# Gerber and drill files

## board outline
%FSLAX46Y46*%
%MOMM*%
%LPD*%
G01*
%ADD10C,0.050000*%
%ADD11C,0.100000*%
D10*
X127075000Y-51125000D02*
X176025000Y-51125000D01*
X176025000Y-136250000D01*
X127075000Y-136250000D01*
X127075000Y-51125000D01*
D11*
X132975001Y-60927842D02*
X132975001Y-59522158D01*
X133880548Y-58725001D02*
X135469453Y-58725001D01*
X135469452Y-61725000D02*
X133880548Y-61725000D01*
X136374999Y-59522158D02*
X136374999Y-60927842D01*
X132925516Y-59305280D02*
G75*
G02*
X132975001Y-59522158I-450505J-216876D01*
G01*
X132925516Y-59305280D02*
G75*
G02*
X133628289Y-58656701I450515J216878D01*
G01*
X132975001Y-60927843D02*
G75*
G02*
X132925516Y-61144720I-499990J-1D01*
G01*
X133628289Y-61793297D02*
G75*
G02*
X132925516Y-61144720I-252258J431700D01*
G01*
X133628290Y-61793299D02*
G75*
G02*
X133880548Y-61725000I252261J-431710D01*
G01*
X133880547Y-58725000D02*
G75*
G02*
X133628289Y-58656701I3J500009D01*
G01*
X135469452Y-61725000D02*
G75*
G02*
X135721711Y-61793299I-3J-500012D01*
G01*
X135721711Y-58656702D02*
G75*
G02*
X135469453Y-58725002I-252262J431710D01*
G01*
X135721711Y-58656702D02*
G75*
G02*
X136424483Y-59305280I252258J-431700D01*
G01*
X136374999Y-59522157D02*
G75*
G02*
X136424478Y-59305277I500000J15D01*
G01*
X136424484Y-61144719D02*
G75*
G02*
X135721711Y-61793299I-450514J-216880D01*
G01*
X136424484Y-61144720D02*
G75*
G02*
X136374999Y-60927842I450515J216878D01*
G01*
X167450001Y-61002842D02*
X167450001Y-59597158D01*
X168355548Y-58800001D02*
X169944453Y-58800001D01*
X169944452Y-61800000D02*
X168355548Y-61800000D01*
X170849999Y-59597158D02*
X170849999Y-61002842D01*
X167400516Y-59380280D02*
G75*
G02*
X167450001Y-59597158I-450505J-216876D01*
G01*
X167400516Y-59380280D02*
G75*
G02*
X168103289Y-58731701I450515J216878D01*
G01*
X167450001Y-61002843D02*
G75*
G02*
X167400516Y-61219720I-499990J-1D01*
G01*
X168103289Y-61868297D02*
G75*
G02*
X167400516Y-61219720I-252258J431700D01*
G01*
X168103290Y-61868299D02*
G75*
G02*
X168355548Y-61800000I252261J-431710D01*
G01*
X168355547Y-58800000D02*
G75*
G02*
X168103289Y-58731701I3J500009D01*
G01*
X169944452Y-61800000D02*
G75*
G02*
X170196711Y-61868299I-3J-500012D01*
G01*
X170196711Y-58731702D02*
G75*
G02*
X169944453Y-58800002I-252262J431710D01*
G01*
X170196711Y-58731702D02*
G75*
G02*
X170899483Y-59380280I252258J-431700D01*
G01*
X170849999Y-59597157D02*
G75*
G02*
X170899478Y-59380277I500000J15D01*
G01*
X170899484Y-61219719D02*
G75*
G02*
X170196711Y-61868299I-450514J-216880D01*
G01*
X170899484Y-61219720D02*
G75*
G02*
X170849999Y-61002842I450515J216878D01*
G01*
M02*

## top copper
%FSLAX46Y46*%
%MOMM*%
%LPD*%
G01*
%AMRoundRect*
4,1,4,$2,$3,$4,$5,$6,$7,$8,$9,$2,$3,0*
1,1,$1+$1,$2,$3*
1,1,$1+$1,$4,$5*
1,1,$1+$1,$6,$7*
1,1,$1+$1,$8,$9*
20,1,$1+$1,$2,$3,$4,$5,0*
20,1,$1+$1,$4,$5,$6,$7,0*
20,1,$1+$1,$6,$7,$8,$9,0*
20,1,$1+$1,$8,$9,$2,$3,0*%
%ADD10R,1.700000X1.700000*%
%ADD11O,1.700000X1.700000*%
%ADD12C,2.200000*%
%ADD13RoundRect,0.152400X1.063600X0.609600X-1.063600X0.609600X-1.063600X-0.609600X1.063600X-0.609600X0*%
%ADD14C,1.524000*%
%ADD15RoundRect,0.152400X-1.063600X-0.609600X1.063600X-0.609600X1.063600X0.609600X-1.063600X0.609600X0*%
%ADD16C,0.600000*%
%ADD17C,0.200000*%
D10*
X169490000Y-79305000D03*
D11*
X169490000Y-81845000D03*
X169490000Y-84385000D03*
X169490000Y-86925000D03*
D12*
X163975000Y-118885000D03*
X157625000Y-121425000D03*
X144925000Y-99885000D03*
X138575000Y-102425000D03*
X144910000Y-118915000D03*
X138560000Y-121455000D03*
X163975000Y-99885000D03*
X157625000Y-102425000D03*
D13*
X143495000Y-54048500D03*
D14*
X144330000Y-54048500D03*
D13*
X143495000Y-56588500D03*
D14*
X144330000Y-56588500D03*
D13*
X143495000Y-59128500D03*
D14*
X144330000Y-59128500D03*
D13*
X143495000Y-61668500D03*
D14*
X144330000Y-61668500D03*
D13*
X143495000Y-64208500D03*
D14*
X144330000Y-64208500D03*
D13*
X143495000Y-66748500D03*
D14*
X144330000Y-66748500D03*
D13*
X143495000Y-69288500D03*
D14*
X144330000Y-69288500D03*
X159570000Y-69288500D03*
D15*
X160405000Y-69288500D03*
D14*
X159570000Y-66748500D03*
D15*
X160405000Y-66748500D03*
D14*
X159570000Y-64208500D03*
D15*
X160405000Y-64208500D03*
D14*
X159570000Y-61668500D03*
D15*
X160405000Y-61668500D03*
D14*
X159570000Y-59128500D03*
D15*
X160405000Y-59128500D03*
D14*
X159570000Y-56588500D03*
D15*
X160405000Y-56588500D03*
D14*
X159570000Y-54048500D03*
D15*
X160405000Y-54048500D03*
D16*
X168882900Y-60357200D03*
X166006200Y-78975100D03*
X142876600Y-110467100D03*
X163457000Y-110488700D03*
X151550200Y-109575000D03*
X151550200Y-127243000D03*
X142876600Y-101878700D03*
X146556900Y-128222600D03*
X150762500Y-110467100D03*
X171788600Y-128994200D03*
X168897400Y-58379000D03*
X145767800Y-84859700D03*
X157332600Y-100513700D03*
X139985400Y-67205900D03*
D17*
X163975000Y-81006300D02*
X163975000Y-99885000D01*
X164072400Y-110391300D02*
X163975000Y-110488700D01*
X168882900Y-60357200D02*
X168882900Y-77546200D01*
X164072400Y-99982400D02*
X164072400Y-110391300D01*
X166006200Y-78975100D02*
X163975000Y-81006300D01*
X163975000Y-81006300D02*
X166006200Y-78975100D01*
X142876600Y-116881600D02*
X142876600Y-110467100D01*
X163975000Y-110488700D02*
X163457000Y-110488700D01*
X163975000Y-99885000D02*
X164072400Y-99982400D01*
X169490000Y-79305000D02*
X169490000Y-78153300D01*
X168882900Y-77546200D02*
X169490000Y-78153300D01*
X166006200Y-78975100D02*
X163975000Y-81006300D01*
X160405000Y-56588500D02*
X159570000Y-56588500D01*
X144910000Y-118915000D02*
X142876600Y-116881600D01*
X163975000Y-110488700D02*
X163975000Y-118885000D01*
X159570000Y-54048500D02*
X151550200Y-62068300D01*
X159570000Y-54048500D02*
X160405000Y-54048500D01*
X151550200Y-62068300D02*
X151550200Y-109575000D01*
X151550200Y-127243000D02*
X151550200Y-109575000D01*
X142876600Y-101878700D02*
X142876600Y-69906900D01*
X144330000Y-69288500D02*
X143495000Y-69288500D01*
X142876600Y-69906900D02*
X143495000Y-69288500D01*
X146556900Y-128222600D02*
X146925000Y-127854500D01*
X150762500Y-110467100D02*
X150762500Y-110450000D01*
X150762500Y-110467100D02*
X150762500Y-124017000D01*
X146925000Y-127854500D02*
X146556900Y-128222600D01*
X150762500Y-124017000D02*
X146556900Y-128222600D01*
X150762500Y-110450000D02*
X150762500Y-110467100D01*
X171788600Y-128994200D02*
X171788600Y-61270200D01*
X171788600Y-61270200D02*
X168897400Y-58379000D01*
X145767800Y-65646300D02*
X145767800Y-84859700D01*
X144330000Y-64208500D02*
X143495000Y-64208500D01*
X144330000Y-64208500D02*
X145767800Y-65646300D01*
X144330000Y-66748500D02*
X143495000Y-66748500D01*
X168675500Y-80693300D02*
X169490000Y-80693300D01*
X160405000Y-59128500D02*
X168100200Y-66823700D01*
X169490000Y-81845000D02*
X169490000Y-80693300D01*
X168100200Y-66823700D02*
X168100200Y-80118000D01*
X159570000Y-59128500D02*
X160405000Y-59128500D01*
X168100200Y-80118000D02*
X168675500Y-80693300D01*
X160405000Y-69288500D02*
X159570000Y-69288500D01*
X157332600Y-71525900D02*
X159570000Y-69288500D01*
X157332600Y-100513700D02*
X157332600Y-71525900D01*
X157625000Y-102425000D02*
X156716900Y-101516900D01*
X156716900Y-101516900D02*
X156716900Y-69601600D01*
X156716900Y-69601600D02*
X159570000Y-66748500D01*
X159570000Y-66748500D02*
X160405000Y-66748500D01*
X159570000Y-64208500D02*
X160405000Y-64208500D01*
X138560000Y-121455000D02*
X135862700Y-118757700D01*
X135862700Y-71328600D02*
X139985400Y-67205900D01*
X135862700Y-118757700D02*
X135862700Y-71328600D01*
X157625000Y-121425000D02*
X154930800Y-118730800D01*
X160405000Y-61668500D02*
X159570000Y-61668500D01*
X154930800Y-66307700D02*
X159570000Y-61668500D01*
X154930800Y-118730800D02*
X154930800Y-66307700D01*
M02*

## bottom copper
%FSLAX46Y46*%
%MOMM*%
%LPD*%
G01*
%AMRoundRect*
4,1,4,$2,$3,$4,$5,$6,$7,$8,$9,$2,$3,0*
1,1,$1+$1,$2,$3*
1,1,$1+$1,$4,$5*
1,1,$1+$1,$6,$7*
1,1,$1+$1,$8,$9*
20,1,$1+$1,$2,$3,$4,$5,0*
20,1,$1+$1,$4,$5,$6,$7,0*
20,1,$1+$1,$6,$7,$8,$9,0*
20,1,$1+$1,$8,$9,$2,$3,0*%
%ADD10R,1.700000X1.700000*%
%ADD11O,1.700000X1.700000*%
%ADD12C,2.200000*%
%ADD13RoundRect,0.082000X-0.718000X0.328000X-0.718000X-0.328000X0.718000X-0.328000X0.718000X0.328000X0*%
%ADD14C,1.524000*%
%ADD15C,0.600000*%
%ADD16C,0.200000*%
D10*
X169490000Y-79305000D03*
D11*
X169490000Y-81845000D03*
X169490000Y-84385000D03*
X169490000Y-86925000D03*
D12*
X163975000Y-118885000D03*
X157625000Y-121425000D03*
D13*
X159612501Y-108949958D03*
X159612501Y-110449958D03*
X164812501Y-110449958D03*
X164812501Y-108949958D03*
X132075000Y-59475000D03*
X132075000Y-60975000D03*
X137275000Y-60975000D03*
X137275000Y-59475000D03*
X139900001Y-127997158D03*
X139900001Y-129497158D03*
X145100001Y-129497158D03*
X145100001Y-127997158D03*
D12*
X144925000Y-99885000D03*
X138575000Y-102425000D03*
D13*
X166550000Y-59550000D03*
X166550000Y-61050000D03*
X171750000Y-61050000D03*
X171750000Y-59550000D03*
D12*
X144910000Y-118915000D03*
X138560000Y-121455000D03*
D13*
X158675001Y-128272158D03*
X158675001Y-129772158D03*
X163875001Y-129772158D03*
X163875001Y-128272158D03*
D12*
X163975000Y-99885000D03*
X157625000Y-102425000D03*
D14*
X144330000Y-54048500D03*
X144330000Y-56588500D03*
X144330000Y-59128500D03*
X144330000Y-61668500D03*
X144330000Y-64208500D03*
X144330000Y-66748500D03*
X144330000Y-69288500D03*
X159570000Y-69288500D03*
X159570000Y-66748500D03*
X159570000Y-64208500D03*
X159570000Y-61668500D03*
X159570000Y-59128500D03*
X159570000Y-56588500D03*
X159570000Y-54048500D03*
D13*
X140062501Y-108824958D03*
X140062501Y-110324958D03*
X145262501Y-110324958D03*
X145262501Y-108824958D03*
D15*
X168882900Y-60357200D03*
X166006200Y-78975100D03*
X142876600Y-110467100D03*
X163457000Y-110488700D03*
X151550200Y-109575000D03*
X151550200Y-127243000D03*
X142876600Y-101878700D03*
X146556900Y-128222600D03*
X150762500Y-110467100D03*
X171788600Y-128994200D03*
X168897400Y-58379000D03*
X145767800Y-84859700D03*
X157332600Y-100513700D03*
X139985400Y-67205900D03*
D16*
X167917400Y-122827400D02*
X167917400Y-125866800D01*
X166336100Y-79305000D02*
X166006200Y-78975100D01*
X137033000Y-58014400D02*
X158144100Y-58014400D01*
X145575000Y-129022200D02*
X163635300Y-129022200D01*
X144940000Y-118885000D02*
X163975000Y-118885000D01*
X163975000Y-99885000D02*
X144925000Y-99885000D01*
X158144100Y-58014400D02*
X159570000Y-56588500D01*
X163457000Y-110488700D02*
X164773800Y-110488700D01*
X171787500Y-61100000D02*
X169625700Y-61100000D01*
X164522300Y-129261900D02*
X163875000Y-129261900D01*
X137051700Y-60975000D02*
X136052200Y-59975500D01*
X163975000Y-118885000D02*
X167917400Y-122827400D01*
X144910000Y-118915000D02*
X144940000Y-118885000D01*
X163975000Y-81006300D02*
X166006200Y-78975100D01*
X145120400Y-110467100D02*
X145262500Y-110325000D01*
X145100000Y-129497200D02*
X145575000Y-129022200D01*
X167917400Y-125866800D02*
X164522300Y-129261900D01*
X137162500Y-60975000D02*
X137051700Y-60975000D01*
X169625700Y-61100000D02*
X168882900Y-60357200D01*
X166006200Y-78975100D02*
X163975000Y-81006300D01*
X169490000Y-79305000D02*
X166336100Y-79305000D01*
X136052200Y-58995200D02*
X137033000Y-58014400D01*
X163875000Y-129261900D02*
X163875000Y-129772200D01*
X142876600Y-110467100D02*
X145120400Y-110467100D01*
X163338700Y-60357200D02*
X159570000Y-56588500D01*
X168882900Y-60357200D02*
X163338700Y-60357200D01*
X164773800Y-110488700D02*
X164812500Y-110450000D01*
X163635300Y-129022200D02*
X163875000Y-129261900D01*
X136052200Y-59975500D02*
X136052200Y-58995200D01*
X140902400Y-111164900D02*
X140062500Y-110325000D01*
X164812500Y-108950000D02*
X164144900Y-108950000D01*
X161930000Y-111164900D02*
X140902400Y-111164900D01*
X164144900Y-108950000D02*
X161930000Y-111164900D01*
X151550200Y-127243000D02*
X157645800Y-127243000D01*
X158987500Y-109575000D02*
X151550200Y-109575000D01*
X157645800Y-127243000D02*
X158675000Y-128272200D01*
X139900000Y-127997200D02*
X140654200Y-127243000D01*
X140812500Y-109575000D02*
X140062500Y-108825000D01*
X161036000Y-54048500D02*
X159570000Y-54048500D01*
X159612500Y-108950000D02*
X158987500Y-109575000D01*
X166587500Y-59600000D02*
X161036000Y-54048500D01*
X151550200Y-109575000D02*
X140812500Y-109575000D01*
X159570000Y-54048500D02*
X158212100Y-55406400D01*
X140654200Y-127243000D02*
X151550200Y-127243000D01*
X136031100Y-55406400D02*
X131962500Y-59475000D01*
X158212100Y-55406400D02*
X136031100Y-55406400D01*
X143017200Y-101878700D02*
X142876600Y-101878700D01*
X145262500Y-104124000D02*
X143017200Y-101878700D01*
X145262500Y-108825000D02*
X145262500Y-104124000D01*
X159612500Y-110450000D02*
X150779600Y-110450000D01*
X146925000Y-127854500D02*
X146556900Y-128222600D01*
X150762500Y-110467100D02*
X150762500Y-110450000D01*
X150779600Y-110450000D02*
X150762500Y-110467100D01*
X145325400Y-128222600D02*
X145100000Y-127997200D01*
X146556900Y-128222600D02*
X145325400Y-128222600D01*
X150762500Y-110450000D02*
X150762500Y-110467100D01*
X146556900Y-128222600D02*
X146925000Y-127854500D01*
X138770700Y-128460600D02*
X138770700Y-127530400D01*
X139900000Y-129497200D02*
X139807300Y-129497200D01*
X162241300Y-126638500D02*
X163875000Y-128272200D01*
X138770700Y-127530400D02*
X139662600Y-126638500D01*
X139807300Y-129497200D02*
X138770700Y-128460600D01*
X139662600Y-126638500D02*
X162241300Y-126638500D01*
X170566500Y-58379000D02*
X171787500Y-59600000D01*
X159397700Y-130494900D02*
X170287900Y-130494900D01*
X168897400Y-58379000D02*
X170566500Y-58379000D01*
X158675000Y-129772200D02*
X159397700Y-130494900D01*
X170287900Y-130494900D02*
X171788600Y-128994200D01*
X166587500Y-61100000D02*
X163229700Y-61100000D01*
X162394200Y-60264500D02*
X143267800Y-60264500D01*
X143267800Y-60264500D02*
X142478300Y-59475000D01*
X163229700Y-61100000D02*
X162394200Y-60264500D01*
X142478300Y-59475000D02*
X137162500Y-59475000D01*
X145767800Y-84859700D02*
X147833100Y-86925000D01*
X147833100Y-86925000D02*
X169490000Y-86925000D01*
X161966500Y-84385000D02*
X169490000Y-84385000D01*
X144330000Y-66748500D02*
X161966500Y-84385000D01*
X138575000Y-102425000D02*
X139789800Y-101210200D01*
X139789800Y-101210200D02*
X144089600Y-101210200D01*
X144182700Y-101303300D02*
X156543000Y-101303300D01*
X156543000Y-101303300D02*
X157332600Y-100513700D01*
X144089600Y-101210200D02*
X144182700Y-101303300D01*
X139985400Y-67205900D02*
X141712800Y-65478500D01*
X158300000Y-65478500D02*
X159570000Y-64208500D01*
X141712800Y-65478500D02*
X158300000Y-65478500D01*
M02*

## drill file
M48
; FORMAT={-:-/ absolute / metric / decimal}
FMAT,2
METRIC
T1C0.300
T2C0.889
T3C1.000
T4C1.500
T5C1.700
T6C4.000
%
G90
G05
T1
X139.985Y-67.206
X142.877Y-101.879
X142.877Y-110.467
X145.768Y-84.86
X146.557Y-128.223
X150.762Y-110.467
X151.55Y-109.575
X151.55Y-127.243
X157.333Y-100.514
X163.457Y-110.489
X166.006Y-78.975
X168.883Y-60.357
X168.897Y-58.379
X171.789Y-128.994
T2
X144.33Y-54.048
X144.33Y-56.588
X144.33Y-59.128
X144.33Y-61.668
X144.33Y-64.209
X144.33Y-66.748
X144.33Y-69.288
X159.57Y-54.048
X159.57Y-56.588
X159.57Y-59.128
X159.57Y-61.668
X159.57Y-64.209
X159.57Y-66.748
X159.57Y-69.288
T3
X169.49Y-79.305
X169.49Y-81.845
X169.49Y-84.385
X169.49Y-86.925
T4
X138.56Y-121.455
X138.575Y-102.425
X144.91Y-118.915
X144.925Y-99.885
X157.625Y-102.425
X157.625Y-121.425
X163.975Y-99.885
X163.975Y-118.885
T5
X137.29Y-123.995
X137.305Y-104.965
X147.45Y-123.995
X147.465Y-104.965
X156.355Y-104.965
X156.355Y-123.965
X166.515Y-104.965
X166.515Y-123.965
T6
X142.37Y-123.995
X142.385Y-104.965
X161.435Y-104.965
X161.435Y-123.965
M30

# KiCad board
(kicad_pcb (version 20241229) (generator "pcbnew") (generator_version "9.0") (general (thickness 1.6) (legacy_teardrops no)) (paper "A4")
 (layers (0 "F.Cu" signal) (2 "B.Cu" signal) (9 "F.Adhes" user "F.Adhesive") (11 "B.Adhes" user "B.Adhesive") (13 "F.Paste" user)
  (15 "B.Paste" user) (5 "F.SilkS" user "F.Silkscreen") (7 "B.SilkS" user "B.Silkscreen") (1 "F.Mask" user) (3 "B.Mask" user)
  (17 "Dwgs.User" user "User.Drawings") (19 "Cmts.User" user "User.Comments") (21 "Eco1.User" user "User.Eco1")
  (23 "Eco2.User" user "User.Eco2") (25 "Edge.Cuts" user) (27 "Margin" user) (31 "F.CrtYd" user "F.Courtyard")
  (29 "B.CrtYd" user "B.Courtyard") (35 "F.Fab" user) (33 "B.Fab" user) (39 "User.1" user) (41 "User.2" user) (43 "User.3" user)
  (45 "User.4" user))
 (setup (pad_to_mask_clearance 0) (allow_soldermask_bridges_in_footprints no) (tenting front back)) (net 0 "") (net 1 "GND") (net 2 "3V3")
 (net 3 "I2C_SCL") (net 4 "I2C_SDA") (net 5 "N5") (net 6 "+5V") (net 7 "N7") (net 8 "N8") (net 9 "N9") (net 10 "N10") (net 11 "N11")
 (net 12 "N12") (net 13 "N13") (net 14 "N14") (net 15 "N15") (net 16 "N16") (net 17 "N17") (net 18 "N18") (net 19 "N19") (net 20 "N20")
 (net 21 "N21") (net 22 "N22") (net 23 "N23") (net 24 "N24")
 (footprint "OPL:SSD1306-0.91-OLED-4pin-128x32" (layer "F.Cu") (at 132.99 77.115)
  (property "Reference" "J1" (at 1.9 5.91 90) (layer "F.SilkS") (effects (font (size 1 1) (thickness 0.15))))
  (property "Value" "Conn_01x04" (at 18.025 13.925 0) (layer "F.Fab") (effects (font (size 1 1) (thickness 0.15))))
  (pad "1" thru_hole rect (at 36.5 2.19) (size 1.7 1.7) (drill 1) (layers "*.Cu" "*.Mask") (remove_unused_layers no) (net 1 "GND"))
  (pad "2" thru_hole oval (at 36.5 4.73) (size 1.7 1.7) (drill 1) (layers "*.Cu" "*.Mask") (remove_unused_layers no) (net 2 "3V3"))
  (pad "3" thru_hole oval (at 36.5 7.27) (size 1.7 1.7) (drill 1) (layers "*.Cu" "*.Mask") (remove_unused_layers no) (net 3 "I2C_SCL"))
  (pad "4" thru_hole oval (at 36.5 9.81) (size 1.7 1.7) (drill 1) (layers "*.Cu" "*.Mask") (remove_unused_layers no) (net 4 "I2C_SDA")))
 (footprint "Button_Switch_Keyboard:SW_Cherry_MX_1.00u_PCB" (layer "F.Cu") (at 163.975 118.885)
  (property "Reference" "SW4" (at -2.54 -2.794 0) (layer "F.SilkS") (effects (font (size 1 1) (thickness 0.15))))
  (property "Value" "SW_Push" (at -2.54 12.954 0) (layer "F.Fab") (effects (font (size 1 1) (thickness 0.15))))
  (pad "" np_thru_hole circle (at -7.62 5.08) (size 1.7 1.7) (drill 1.7) (layers "*.Cu" "*.Mask"))
  (pad "" np_thru_hole circle (at -2.54 5.08) (size 4 4) (drill 4) (layers "*.Cu" "*.Mask"))
  (pad "" np_thru_hole circle (at 2.54 5.08) (size 1.7 1.7) (drill 1.7) (layers "*.Cu" "*.Mask"))
  (pad "1" thru_hole circle (at 0 0) (size 2.2 2.2) (drill 1.5) (layers "*.Cu" "*.Mask") (remove_unused_layers no) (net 1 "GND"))
  (pad "2" thru_hole circle (at -6.35 2.54) (size 2.2 2.2) (drill 1.5) (layers "*.Cu" "*.Mask") (remove_unused_layers no) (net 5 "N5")))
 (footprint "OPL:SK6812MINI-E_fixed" (layer "F.Cu") (at 162.2125 109.8028)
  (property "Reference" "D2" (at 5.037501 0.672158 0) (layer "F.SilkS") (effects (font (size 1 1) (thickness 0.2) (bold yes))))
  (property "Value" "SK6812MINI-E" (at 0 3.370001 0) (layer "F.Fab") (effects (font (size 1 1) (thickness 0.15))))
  (pad "1" smd roundrect (at -2.599999 -0.852842 270) (size 0.82 1.6) (layers "B.Cu" "B.Mask" "B.Paste") (roundrect_rratio 0.1)
   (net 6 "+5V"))
  (pad "2" smd roundrect (at -2.599999 0.647158 270) (size 0.82 1.6) (layers "B.Cu" "B.Mask" "B.Paste") (roundrect_rratio 0.1) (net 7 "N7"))
  (pad "3" smd roundrect (at 2.600001 0.647158 270) (size 0.82 1.6) (layers "B.Cu" "B.Mask" "B.Paste") (roundrect_rratio 0.1) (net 1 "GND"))
  (pad "4" smd roundrect (at 2.600001 -0.852842 270) (size 0.82 1.6) (layers "B.Cu" "B.Mask" "B.Paste") (roundrect_rratio 0.1) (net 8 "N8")))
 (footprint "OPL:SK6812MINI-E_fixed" (layer "F.Cu") (at 134.674999 60.327842)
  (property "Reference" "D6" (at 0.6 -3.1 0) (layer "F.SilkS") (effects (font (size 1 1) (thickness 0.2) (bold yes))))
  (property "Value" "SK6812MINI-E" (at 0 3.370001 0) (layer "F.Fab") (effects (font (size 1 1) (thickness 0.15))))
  (fp_line (start -1.699998 0.6) (end -1.699998 -0.805684) (stroke (width 0.1) (type solid)) (layer "Edge.Cuts"))
  (fp_line (start -0.794451 -1.602841) (end 0.794454 -1.602841) (stroke (width 0.1) (type solid)) (layer "Edge.Cuts"))
  (fp_line (start 0.794453 1.397158) (end -0.794451 1.397158) (stroke (width 0.1) (type solid)) (layer "Edge.Cuts"))
  (fp_line (start 1.7 -0.805684) (end 1.7 0.6) (stroke (width 0.1) (type solid)) (layer "Edge.Cuts"))
  (fp_arc (start -1.749483 -1.022562) (mid -1.712526 -0.91691) (end -1.699998 -0.805684) (stroke (width 0.1) (type solid))
   (layer "Edge.Cuts"))
  (fp_arc (start -1.749483 -1.022562) (mid -1.63807 -1.606877) (end -1.04671 -1.671141) (stroke (width 0.1) (type solid))
   (layer "Edge.Cuts"))
  (fp_arc (start -1.699998 0.600001) (mid -1.712526 0.711226) (end -1.749483 0.816878) (stroke (width 0.1) (type solid)) (layer "Edge.Cuts"))
  (fp_arc (start -1.04671 1.465455) (mid -1.638069 1.401192) (end -1.749483 0.816878) (stroke (width 0.1) (type solid)) (layer "Edge.Cuts"))
  (fp_arc (start -1.046709 1.465457) (mid -0.925121 1.414535) (end -0.794451 1.397158) (stroke (width 0.1) (type solid)) (layer "Edge.Cuts"))
  (fp_arc (start -0.794452 -1.602842) (mid -0.925122 -1.620219) (end -1.04671 -1.671141) (stroke (width 0.1) (type solid))
   (layer "Edge.Cuts"))
  (fp_arc (start 0.794453 1.397158) (mid 0.925124 1.414535) (end 1.046712 1.465457) (stroke (width 0.1) (type solid)) (layer "Edge.Cuts"))
  (fp_arc (start 1.046712 -1.67114) (mid 0.925124 -1.620218) (end 0.794454 -1.602841) (stroke (width 0.1) (type solid)) (layer "Edge.Cuts"))
  (fp_arc (start 1.046712 -1.67114) (mid 1.638072 -1.606876) (end 1.749485 -1.022562) (stroke (width 0.1) (type solid)) (layer "Edge.Cuts"))
  (fp_arc (start 1.7 -0.805685) (mid 1.712528 -0.91691) (end 1.749485 -1.022562) (stroke (width 0.1) (type solid)) (layer "Edge.Cuts"))
  (fp_arc (start 1.749485 0.816877) (mid 1.638073 1.401193) (end 1.046712 1.465457) (stroke (width 0.1) (type solid)) (layer "Edge.Cuts"))
  (fp_arc (start 1.749485 0.816878) (mid 1.712528 0.711226) (end 1.7 0.6) (stroke (width 0.1) (type solid)) (layer "Edge.Cuts"))
  (pad "1" smd roundrect (at -2.599999 -0.852842 270) (size 0.82 1.6) (layers "B.Cu" "B.Mask" "B.Paste") (roundrect_rratio 0.1)
   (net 6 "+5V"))
  (pad "2" smd roundrect (at -2.599999 0.647158 270) (size 0.82 1.6) (layers "B.Cu" "B.Mask" "B.Paste") (roundrect_rratio 0.1) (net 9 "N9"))
  (pad "3" smd roundrect (at 2.600001 0.647158 270) (size 0.82 1.6) (layers "B.Cu" "B.Mask" "B.Paste") (roundrect_rratio 0.1) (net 1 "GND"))
  (pad "4" smd roundrect (at 2.600001 -0.852842 270) (size 0.82 1.6) (layers "B.Cu" "B.Mask" "B.Paste") (roundrect_rratio 0.1)
   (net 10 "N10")))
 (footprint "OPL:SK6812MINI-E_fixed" (layer "F.Cu") (at 142.5 128.85)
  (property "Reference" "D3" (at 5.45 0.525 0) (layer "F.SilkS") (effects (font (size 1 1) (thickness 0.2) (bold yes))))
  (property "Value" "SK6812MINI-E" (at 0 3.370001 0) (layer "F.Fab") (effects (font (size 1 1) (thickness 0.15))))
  (pad "1" smd roundrect (at -2.599999 -0.852842 270) (size 0.82 1.6) (layers "B.Cu" "B.Mask" "B.Paste") (roundrect_rratio 0.1)
   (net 6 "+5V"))
  (pad "2" smd roundrect (at -2.599999 0.647158 270) (size 0.82 1.6) (layers "B.Cu" "B.Mask" "B.Paste") (roundrect_rratio 0.1)
   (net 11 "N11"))
  (pad "3" smd roundrect (at 2.600001 0.647158 270) (size 0.82 1.6) (layers "B.Cu" "B.Mask" "B.Paste") (roundrect_rratio 0.1) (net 1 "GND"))
  (pad "4" smd roundrect (at 2.600001 -0.852842 270) (size 0.82 1.6) (layers "B.Cu" "B.Mask" "B.Paste") (roundrect_rratio 0.1) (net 7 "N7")))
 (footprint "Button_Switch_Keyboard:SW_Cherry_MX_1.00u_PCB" (layer "F.Cu") (at 144.925 99.885)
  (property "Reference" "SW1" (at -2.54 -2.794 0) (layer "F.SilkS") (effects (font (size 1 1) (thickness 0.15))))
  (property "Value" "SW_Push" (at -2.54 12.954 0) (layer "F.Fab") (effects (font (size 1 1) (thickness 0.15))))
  (pad "" np_thru_hole circle (at -7.62 5.08) (size 1.7 1.7) (drill 1.7) (layers "*.Cu" "*.Mask"))
  (pad "" np_thru_hole circle (at -2.54 5.08) (size 4 4) (drill 4) (layers "*.Cu" "*.Mask"))
  (pad "" np_thru_hole circle (at 2.54 5.08) (size 1.7 1.7) (drill 1.7) (layers "*.Cu" "*.Mask"))
  (pad "1" thru_hole circle (at 0 0) (size 2.2 2.2) (drill 1.5) (layers "*.Cu" "*.Mask") (remove_unused_layers no) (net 1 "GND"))
  (pad "2" thru_hole circle (at -6.35 2.54) (size 2.2 2.2) (drill 1.5) (layers "*.Cu" "*.Mask") (remove_unused_layers no) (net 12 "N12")))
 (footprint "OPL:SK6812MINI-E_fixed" (layer "F.Cu") (at 169.149999 60.402842)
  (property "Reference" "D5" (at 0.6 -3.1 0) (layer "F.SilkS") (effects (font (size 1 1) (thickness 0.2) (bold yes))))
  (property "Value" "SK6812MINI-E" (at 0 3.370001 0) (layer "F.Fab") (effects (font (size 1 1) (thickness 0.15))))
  (fp_line (start -1.699998 0.6) (end -1.699998 -0.805684) (stroke (width 0.1) (type solid)) (layer "Edge.Cuts"))
  (fp_line (start -0.794451 -1.602841) (end 0.794454 -1.602841) (stroke (width 0.1) (type solid)) (layer "Edge.Cuts"))
  (fp_line (start 0.794453 1.397158) (end -0.794451 1.397158) (stroke (width 0.1) (type solid)) (layer "Edge.Cuts"))
  (fp_line (start 1.7 -0.805684) (end 1.7 0.6) (stroke (width 0.1) (type solid)) (layer "Edge.Cuts"))
  (fp_arc (start -1.749483 -1.022562) (mid -1.712526 -0.91691) (end -1.699998 -0.805684) (stroke (width 0.1) (type solid))
   (layer "Edge.Cuts"))
  (fp_arc (start -1.749483 -1.022562) (mid -1.63807 -1.606877) (end -1.04671 -1.671141) (stroke (width 0.1) (type solid))
   (layer "Edge.Cuts"))
  (fp_arc (start -1.699998 0.600001) (mid -1.712526 0.711226) (end -1.749483 0.816878) (stroke (width 0.1) (type solid)) (layer "Edge.Cuts"))
  (fp_arc (start -1.04671 1.465455) (mid -1.638069 1.401192) (end -1.749483 0.816878) (stroke (width 0.1) (type solid)) (layer "Edge.Cuts"))
  (fp_arc (start -1.046709 1.465457) (mid -0.925121 1.414535) (end -0.794451 1.397158) (stroke (width 0.1) (type solid)) (layer "Edge.Cuts"))
  (fp_arc (start -0.794452 -1.602842) (mid -0.925122 -1.620219) (end -1.04671 -1.671141) (stroke (width 0.1) (type solid))
   (layer "Edge.Cuts"))
  (fp_arc (start 0.794453 1.397158) (mid 0.925124 1.414535) (end 1.046712 1.465457) (stroke (width 0.1) (type solid)) (layer "Edge.Cuts"))
  (fp_arc (start 1.046712 -1.67114) (mid 0.925124 -1.620218) (end 0.794454 -1.602841) (stroke (width 0.1) (type solid)) (layer "Edge.Cuts"))
  (fp_arc (start 1.046712 -1.67114) (mid 1.638072 -1.606876) (end 1.749485 -1.022562) (stroke (width 0.1) (type solid)) (layer "Edge.Cuts"))
  (fp_arc (start 1.7 -0.805685) (mid 1.712528 -0.91691) (end 1.749485 -1.022562) (stroke (width 0.1) (type solid)) (layer "Edge.Cuts"))
  (fp_arc (start 1.749485 0.816877) (mid 1.638073 1.401193) (end 1.046712 1.465457) (stroke (width 0.1) (type solid)) (layer "Edge.Cuts"))
  (fp_arc (start 1.749485 0.816878) (mid 1.712528 0.711226) (end 1.7 0.6) (stroke (width 0.1) (type solid)) (layer "Edge.Cuts"))
  (pad "1" smd roundrect (at -2.599999 -0.852842 270) (size 0.82 1.6) (layers "B.Cu" "B.Mask" "B.Paste") (roundrect_rratio 0.1)
   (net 6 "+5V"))
  (pad "2" smd roundrect (at -2.599999 0.647158 270) (size 0.82 1.6) (layers "B.Cu" "B.Mask" "B.Paste") (roundrect_rratio 0.1)
   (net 10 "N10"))
  (pad "3" smd roundrect (at 2.600001 0.647158 270) (size 0.82 1.6) (layers "B.Cu" "B.Mask" "B.Paste") (roundrect_rratio 0.1) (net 1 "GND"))
  (pad "4" smd roundrect (at 2.600001 -0.852842 270) (size 0.82 1.6) (layers "B.Cu" "B.Mask" "B.Paste") (roundrect_rratio 0.1)
   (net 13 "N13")))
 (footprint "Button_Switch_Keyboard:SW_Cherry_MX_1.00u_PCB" (layer "F.Cu") (at 144.91 118.915)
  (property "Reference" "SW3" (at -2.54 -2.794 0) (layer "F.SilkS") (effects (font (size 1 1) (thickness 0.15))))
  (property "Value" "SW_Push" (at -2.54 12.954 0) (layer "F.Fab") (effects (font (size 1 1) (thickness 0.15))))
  (pad "" np_thru_hole circle (at -7.62 5.08) (size 1.7 1.7) (drill 1.7) (layers "*.Cu" "*.Mask"))
  (pad "" np_thru_hole circle (at -2.54 5.08) (size 4 4) (drill 4) (layers "*.Cu" "*.Mask"))
  (pad "" np_thru_hole circle (at 2.54 5.08) (size 1.7 1.7) (drill 1.7) (layers "*.Cu" "*.Mask"))
  (pad "1" thru_hole circle (at 0 0) (size 2.2 2.2) (drill 1.5) (layers "*.Cu" "*.Mask") (remove_unused_layers no) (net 1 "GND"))
  (pad "2" thru_hole circle (at -6.35 2.54) (size 2.2 2.2) (drill 1.5) (layers "*.Cu" "*.Mask") (remove_unused_layers no) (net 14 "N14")))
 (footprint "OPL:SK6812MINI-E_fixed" (layer "F.Cu") (at 161.275 129.125)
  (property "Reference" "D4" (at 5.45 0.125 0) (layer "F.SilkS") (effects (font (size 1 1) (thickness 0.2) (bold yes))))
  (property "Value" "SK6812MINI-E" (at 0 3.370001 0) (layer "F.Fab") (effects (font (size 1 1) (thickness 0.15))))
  (pad "1" smd roundrect (at -2.599999 -0.852842 270) (size 0.82 1.6) (layers "B.Cu" "B.Mask" "B.Paste") (roundrect_rratio 0.1)
   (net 6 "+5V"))
  (pad "2" smd roundrect (at -2.599999 0.647158 270) (size 0.82 1.6) (layers "B.Cu" "B.Mask" "B.Paste") (roundrect_rratio 0.1)
   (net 13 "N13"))
  (pad "3" smd roundrect (at 2.600001 0.647158 270) (size 0.82 1.6) (layers "B.Cu" "B.Mask" "B.Paste") (roundrect_rratio 0.1) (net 1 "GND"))
  (pad "4" smd roundrect (at 2.600001 -0.852842 270) (size 0.82 1.6) (layers "B.Cu" "B.Mask" "B.Paste") (roundrect_rratio 0.1)
   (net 11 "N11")))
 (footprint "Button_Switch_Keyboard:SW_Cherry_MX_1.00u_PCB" (layer "F.Cu") (at 163.975 99.885)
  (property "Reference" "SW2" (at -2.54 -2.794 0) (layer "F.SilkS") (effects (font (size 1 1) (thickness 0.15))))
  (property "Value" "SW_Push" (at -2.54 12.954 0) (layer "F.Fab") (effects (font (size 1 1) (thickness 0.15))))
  (pad "" np_thru_hole circle (at -7.62 5.08) (size 1.7 1.7) (drill 1.7) (layers "*.Cu" "*.Mask"))
  (pad "" np_thru_hole circle (at -2.54 5.08) (size 4 4) (drill 4) (layers "*.Cu" "*.Mask"))
  (pad "" np_thru_hole circle (at 2.54 5.08) (size 1.7 1.7) (drill 1.7) (layers "*.Cu" "*.Mask"))
  (pad "1" thru_hole circle (at 0 0) (size 2.2 2.2) (drill 1.5) (layers "*.Cu" "*.Mask") (remove_unused_layers no) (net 1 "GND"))
  (pad "2" thru_hole circle (at -6.35 2.54) (size 2.2 2.2) (drill 1.5) (layers "*.Cu" "*.Mask") (remove_unused_layers no) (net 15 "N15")))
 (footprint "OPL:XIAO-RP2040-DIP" (layer "F.Cu") (at 151.95 61.6685)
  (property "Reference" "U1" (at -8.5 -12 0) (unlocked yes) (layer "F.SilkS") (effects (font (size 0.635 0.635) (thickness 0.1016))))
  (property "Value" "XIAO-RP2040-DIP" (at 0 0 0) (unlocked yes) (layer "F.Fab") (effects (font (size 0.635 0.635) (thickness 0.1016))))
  (pad "1" smd roundrect (at -8.455 -7.62 180) (size 2.432 1.524) (layers "F.Cu" "F.Mask") (roundrect_rratio 0.1) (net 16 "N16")
   (thermal_bridge_angle 45))
  (pad "1" thru_hole circle (at -7.62 -7.62 180) (size 1.524 1.524) (drill 0.889) (layers "*.Cu" "*.Mask") (remove_unused_layers no)
   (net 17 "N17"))
  (pad "2" smd roundrect (at -8.455 -5.08 180) (size 2.432 1.524) (layers "F.Cu" "F.Mask") (roundrect_rratio 0.1) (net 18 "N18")
   (thermal_bridge_angle 45))
  (pad "2" thru_hole circle (at -7.62 -5.08 180) (size 1.524 1.524) (drill 0.889) (layers "*.Cu" "*.Mask") (remove_unused_layers no)
   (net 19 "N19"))
  (pad "3" smd roundrect (at -8.455 -2.54 180) (size 2.432 1.524) (layers "F.Cu" "F.Mask") (roundrect_rratio 0.1) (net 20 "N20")
   (thermal_bridge_angle 45))
  (pad "3" thru_hole circle (at -7.62 -2.54 180) (size 1.524 1.524) (drill 0.889) (layers "*.Cu" "*.Mask") (remove_unused_layers no)
   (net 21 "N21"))
  (pad "4" smd roundrect (at -8.455 0 180) (size 2.432 1.524) (layers "F.Cu" "F.Mask") (roundrect_rratio 0.1) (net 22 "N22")
   (thermal_bridge_angle 45))
  (pad "4" thru_hole circle (at -7.62 0 180) (size 1.524 1.524) (drill 0.889) (layers "*.Cu" "*.Mask") (remove_unused_layers no)
   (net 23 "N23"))
  (pad "5" smd roundrect (at -8.455 2.54 180) (size 2.432 1.524) (layers "F.Cu" "F.Mask") (roundrect_rratio 0.1) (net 4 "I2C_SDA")
   (thermal_bridge_angle 45))
  (pad "5" thru_hole circle (at -7.62 2.54 180) (size 1.524 1.524) (drill 0.889) (layers "*.Cu" "*.Mask") (remove_unused_layers no)
   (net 4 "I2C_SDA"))
  (pad "6" smd roundrect (at -8.455 5.08 180) (size 2.432 1.524) (layers "F.Cu" "F.Mask") (roundrect_rratio 0.1) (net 3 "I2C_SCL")
   (thermal_bridge_angle 45))
  (pad "6" thru_hole circle (at -7.62 5.08 180) (size 1.524 1.524) (drill 0.889) (layers "*.Cu" "*.Mask") (remove_unused_layers no)
   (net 3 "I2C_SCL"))
  (pad "7" smd roundrect (at -8.455 7.62 180) (size 2.432 1.524) (layers "F.Cu" "F.Mask") (roundrect_rratio 0.1) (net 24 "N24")
   (thermal_bridge_angle 45))
  (pad "7" thru_hole circle (at -7.62 7.62 180) (size 1.524 1.524) (drill 0.889) (layers "*.Cu" "*.Mask") (remove_unused_layers no)
   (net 24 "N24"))
  (pad "8" thru_hole circle (at 7.62 7.62) (size 1.524 1.524) (drill 0.889) (layers "*.Cu" "*.Mask") (remove_unused_layers no)
   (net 12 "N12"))
  (pad "8" smd roundrect (at 8.455 7.62) (size 2.432 1.524) (layers "F.Cu" "F.Mask") (roundrect_rratio 0.1) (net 12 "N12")
   (thermal_bridge_angle 45))
  (pad "9" thru_hole circle (at 7.62 5.08) (size 1.524 1.524) (drill 0.889) (layers "*.Cu" "*.Mask") (remove_unused_layers no)
   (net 15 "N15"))
  (pad "9" smd roundrect (at 8.455 5.08) (size 2.432 1.524) (layers "F.Cu" "F.Mask") (roundrect_rratio 0.1) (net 15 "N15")
   (thermal_bridge_angle 45))
  (pad "10" thru_hole circle (at 7.62 2.54) (size 1.524 1.524) (drill 0.889) (layers "*.Cu" "*.Mask") (remove_unused_layers no)
   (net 14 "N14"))
  (pad "10" smd roundrect (at 8.455 2.54) (size 2.432 1.524) (layers "F.Cu" "F.Mask") (roundrect_rratio 0.1) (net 14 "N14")
   (thermal_bridge_angle 45))
  (pad "11" thru_hole circle (at 7.62 0) (size 1.524 1.524) (drill 0.889) (layers "*.Cu" "*.Mask") (remove_unused_layers no) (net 5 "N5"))
  (pad "11" smd roundrect (at 8.455 0) (size 2.432 1.524) (layers "F.Cu" "F.Mask") (roundrect_rratio 0.1) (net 5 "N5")
   (thermal_bridge_angle 45))
  (pad "12" thru_hole circle (at 7.62 -2.54) (size 1.524 1.524) (drill 0.889) (layers "*.Cu" "*.Mask") (remove_unused_layers no)
   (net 2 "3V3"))
  (pad "12" smd roundrect (at 8.455 -2.54) (size 2.432 1.524) (layers "F.Cu" "F.Mask") (roundrect_rratio 0.1) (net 2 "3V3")
   (thermal_bridge_angle 45))
  (pad "13" thru_hole circle (at 7.62 -5.08) (size 1.524 1.524) (drill 0.889) (layers "*.Cu" "*.Mask") (remove_unused_layers no)
   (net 1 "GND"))
  (pad "13" smd roundrect (at 8.455 -5.08) (size 2.432 1.524) (layers "F.Cu" "F.Mask") (roundrect_rratio 0.1) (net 1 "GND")
   (thermal_bridge_angle 45))
  (pad "14" thru_hole circle (at 7.62 -7.62) (size 1.524 1.524) (drill 0.889) (layers "*.Cu" "*.Mask") (remove_unused_layers no)
   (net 6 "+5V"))
  (pad "14" smd roundrect (at 8.455 -7.62) (size 2.432 1.524) (layers "F.Cu" "F.Mask") (roundrect_rratio 0.1) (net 6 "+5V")
   (thermal_bridge_angle 45)))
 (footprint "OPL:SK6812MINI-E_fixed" (layer "F.Cu") (at 142.6625 109.6778)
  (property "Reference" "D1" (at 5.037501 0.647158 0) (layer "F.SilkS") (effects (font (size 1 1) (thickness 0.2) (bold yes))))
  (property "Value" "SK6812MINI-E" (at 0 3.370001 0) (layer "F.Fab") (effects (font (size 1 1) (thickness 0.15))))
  (pad "1" smd roundrect (at -2.599999 -0.852842 270) (size 0.82 1.6) (layers "B.Cu" "B.Mask" "B.Paste") (roundrect_rratio 0.1)
   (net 6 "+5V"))
  (pad "2" smd roundrect (at -2.599999 0.647158 270) (size 0.82 1.6) (layers "B.Cu" "B.Mask" "B.Paste") (roundrect_rratio 0.1) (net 8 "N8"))
  (pad "3" smd roundrect (at 2.600001 0.647158 270) (size 0.82 1.6) (layers "B.Cu" "B.Mask" "B.Paste") (roundrect_rratio 0.1) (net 1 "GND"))
  (pad "4" smd roundrect (at 2.600001 -0.852842 270) (size 0.82 1.6) (layers "B.Cu" "B.Mask" "B.Paste") (roundrect_rratio 0.1)
   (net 24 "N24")))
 (gr_rect (start 127.075 51.125) (end 176.025 136.25) (stroke (width 0.05) (type default)) (fill no) (layer "Edge.Cuts"))
 (segment (start 163.975 81.0063) (end 163.975 99.885) (width 0.2) (layer "F.Cu") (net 1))
 (segment (start 164.0724 110.3913) (end 163.975 110.4887) (width 0.2) (layer "F.Cu") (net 1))
 (segment (start 168.8829 60.3572) (end 168.8829 77.5462) (width 0.2) (layer "F.Cu") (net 1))
 (segment (start 164.0724 99.9824) (end 164.0724 110.3913) (width 0.2) (layer "F.Cu") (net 1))
 (segment (start 166.0062 78.9751) (end 163.975 81.0063) (width 0.2) (layer "F.Cu") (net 1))
 (segment (start 163.975 81.0063) (end 166.0062 78.9751) (width 0.2) (layer "F.Cu") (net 1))
 (segment (start 142.8766 116.8816) (end 142.8766 110.4671) (width 0.2) (layer "F.Cu") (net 1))
 (segment (start 163.975 110.4887) (end 163.457 110.4887) (width 0.2) (layer "F.Cu") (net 1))
 (segment (start 163.975 99.885) (end 164.0724 99.9824) (width 0.2) (layer "F.Cu") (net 1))
 (segment (start 169.49 79.305) (end 169.49 78.1533) (width 0.2) (layer "F.Cu") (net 1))
 (segment (start 168.8829 77.5462) (end 169.49 78.1533) (width 0.2) (layer "F.Cu") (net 1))
 (segment (start 166.0062 78.9751) (end 163.975 81.0063) (width 0.2) (layer "F.Cu") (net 1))
 (segment (start 160.405 56.5885) (end 159.57 56.5885) (width 0.2) (layer "F.Cu") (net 1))
 (segment (start 144.91 118.915) (end 142.8766 116.8816) (width 0.2) (layer "F.Cu") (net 1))
 (segment (start 163.975 110.4887) (end 163.975 118.885) (width 0.2) (layer "F.Cu") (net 1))
 (via (at 168.8829 60.3572) (size 0.6) (drill 0.3) (layers "F.Cu" "B.Cu") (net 1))
 (via (at 166.0062 78.9751) (size 0.6) (drill 0.3) (layers "F.Cu" "B.Cu") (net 1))
 (via (at 142.8766 110.4671) (size 0.6) (drill 0.3) (layers "F.Cu" "B.Cu") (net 1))
 (via (at 163.457 110.4887) (size 0.6) (drill 0.3) (layers "F.Cu" "B.Cu") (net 1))
 (segment (start 167.9174 122.8274) (end 167.9174 125.8668) (width 0.2) (layer "B.Cu") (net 1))
 (segment (start 166.3361 79.305) (end 166.0062 78.9751) (width 0.2) (layer "B.Cu") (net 1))
 (segment (start 137.033 58.0144) (end 158.1441 58.0144) (width 0.2) (layer "B.Cu") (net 1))
 (segment (start 145.575 129.0222) (end 163.6353 129.0222) (width 0.2) (layer "B.Cu") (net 1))
 (segment (start 144.94 118.885) (end 163.975 118.885) (width 0.2) (layer "B.Cu") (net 1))
 (segment (start 163.975 99.885) (end 144.925 99.885) (width 0.2) (layer "B.Cu") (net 1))
 (segment (start 158.1441 58.0144) (end 159.57 56.5885) (width 0.2) (layer "B.Cu") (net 1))
 (segment (start 163.457 110.4887) (end 164.7738 110.4887) (width 0.2) (layer "B.Cu") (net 1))
 (segment (start 171.7875 61.1) (end 169.6257 61.1) (width 0.2) (layer "B.Cu") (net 1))
 (segment (start 164.5223 129.2619) (end 163.875 129.2619) (width 0.2) (layer "B.Cu") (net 1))
 (segment (start 137.0517 60.975) (end 136.0522 59.9755) (width 0.2) (layer "B.Cu") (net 1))
 (segment (start 163.975 118.885) (end 167.9174 122.8274) (width 0.2) (layer "B.Cu") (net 1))
 (segment (start 144.91 118.915) (end 144.94 118.885) (width 0.2) (layer "B.Cu") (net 1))
 (segment (start 163.975 81.0063) (end 166.0062 78.9751) (width 0.2) (layer "B.Cu") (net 1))
 (segment (start 145.1204 110.4671) (end 145.2625 110.325) (width 0.2) (layer "B.Cu") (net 1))
 (segment (start 145.1 129.4972) (end 145.575 129.0222) (width 0.2) (layer "B.Cu") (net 1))
 (segment (start 167.9174 125.8668) (end 164.5223 129.2619) (width 0.2) (layer "B.Cu") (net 1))
 (segment (start 137.1625 60.975) (end 137.0517 60.975) (width 0.2) (layer "B.Cu") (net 1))
 (segment (start 169.6257 61.1) (end 168.8829 60.3572) (width 0.2) (layer "B.Cu") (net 1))
 (segment (start 166.0062 78.9751) (end 163.975 81.0063) (width 0.2) (layer "B.Cu") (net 1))
 (segment (start 169.49 79.305) (end 166.3361 79.305) (width 0.2) (layer "B.Cu") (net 1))
 (segment (start 136.0522 58.9952) (end 137.033 58.0144) (width 0.2) (layer "B.Cu") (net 1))
 (segment (start 163.875 129.2619) (end 163.875 129.7722) (width 0.2) (layer "B.Cu") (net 1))
 (segment (start 142.8766 110.4671) (end 145.1204 110.4671) (width 0.2) (layer "B.Cu") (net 1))
 (segment (start 163.3387 60.3572) (end 159.57 56.5885) (width 0.2) (layer "B.Cu") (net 1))
 (segment (start 168.8829 60.3572) (end 163.3387 60.3572) (width 0.2) (layer "B.Cu") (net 1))
 (segment (start 164.7738 110.4887) (end 164.8125 110.45) (width 0.2) (layer "B.Cu") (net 1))
 (segment (start 163.6353 129.0222) (end 163.875 129.2619) (width 0.2) (layer "B.Cu") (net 1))
 (segment (start 136.0522 59.9755) (end 136.0522 58.9952) (width 0.2) (layer "B.Cu") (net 1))
 (segment (start 140.9024 111.1649) (end 140.0625 110.325) (width 0.2) (layer "B.Cu") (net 8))
 (segment (start 164.8125 108.95) (end 164.1449 108.95) (width 0.2) (layer "B.Cu") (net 8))
 (segment (start 161.93 111.1649) (end 140.9024 111.1649) (width 0.2) (layer "B.Cu") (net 8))
 (segment (start 164.1449 108.95) (end 161.93 111.1649) (width 0.2) (layer "B.Cu") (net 8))
 (segment (start 159.57 54.0485) (end 151.5502 62.0683) (width 0.2) (layer "F.Cu") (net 6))
 (segment (start 159.57 54.0485) (end 160.405 54.0485) (width 0.2) (layer "F.Cu") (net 6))
 (segment (start 151.5502 62.0683) (end 151.5502 109.575) (width 0.2) (layer "F.Cu") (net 6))
 (segment (start 151.5502 127.243) (end 151.5502 109.575) (width 0.2) (layer "F.Cu") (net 6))
 (via (at 151.5502 109.575) (size 0.6) (drill 0.3) (layers "F.Cu" "B.Cu") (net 6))
 (via (at 151.5502 127.243) (size 0.6) (drill 0.3) (layers "F.Cu" "B.Cu") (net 6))
 (segment (start 151.5502 127.243) (end 157.6458 127.243) (width 0.2) (layer "B.Cu") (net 6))
 (segment (start 158.9875 109.575) (end 151.5502 109.575) (width 0.2) (layer "B.Cu") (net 6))
 (segment (start 157.6458 127.243) (end 158.675 128.2722) (width 0.2) (layer "B.Cu") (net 6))
 (segment (start 139.9 127.9972) (end 140.6542 127.243) (width 0.2) (layer "B.Cu") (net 6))
 (segment (start 140.8125 109.575) (end 140.0625 108.825) (width 0.2) (layer "B.Cu") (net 6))
 (segment (start 161.036 54.0485) (end 159.57 54.0485) (width 0.2) (layer "B.Cu") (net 6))
 (segment (start 159.6125 108.95) (end 158.9875 109.575) (width 0.2) (layer "B.Cu") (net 6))
 (segment (start 166.5875 59.6) (end 161.036 54.0485) (width 0.2) (layer "B.Cu") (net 6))
 (segment (start 151.5502 109.575) (end 140.8125 109.575) (width 0.2) (layer "B.Cu") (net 6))
 (segment (start 159.57 54.0485) (end 158.2121 55.4064) (width 0.2) (layer "B.Cu") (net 6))
 (segment (start 140.6542 127.243) (end 151.5502 127.243) (width 0.2) (layer "B.Cu") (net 6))
 (segment (start 136.0311 55.4064) (end 131.9625 59.475) (width 0.2) (layer "B.Cu") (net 6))
 (segment (start 158.2121 55.4064) (end 136.0311 55.4064) (width 0.2) (layer "B.Cu") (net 6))
 (segment (start 142.8766 101.8787) (end 142.8766 69.9069) (width 0.2) (layer "F.Cu") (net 24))
 (segment (start 144.33 69.2885) (end 143.495 69.2885) (width 0.2) (layer "F.Cu") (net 24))
 (segment (start 142.8766 69.9069) (end 143.495 69.2885) (width 0.2) (layer "F.Cu") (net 24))
 (via (at 142.8766 101.8787) (size 0.6) (drill 0.3) (layers "F.Cu" "B.Cu") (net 24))
 (segment (start 143.0172 101.8787) (end 142.8766 101.8787) (width 0.2) (layer "B.Cu") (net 24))
 (segment (start 145.2625 104.124) (end 143.0172 101.8787) (width 0.2) (layer "B.Cu") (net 24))
 (segment (start 145.2625 108.825) (end 145.2625 104.124) (width 0.2) (layer "B.Cu") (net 24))
 (segment (start 146.5569 128.2226) (end 146.925 127.8545) (width 0.2) (layer "F.Cu") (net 7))
 (segment (start 150.7625 110.4671) (end 150.7625 110.45) (width 0.2) (layer "F.Cu") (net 7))
 (segment (start 150.7625 110.4671) (end 150.7625 124.017) (width 0.2) (layer "F.Cu") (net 7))
 (segment (start 146.925 127.8545) (end 146.5569 128.2226) (width 0.2) (layer "F.Cu") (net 7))
 (segment (start 150.7625 124.017) (end 146.5569 128.2226) (width 0.2) (layer "F.Cu") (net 7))
 (segment (start 150.7625 110.45) (end 150.7625 110.4671) (width 0.2) (layer "F.Cu") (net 7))
 (via (at 146.5569 128.2226) (size 0.6) (drill 0.3) (layers "F.Cu" "B.Cu") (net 7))
 (via (at 150.7625 110.4671) (size 0.6) (drill 0.3) (layers "F.Cu" "B.Cu") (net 7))
 (segment (start 159.6125 110.45) (end 150.7796 110.45) (width 0.2) (layer "B.Cu") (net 7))
 (segment (start 146.925 127.8545) (end 146.5569 128.2226) (width 0.2) (layer "B.Cu") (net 7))
 (segment (start 150.7625 110.4671) (end 150.7625 110.45) (width 0.2) (layer "B.Cu") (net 7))
 (segment (start 150.7796 110.45) (end 150.7625 110.4671) (width 0.2) (layer "B.Cu") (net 7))
 (segment (start 145.3254 128.2226) (end 145.1 127.9972) (width 0.2) (layer "B.Cu") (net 7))
 (segment (start 146.5569 128.2226) (end 145.3254 128.2226) (width 0.2) (layer "B.Cu") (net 7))
 (segment (start 150.7625 110.45) (end 150.7625 110.4671) (width 0.2) (layer "B.Cu") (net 7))
 (segment (start 146.5569 128.2226) (end 146.925 127.8545) (width 0.2) (layer "B.Cu") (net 7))
 (segment (start 138.7707 128.4606) (end 138.7707 127.5304) (width 0.2) (layer "B.Cu") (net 11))
 (segment (start 139.9 129.4972) (end 139.8073 129.4972) (width 0.2) (layer "B.Cu") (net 11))
 (segment (start 162.2413 126.6385) (end 163.875 128.2722) (width 0.2) (layer "B.Cu") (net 11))
 (segment (start 138.7707 127.5304) (end 139.6626 126.6385) (width 0.2) (layer "B.Cu") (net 11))
 (segment (start 139.8073 129.4972) (end 138.7707 128.4606) (width 0.2) (layer "B.Cu") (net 11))
 (segment (start 139.6626 126.6385) (end 162.2413 126.6385) (width 0.2) (layer "B.Cu") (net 11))
 (segment (start 171.7886 128.9942) (end 171.7886 61.2702) (width 0.2) (layer "F.Cu") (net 13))
 (segment (start 171.7886 61.2702) (end 168.8974 58.379) (width 0.2) (layer "F.Cu") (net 13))
 (via (at 171.7886 128.9942) (size 0.6) (drill 0.3) (layers "F.Cu" "B.Cu") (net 13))
 (via (at 168.8974 58.379) (size 0.6) (drill 0.3) (layers "F.Cu" "B.Cu") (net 13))
 (segment (start 170.5665 58.379) (end 171.7875 59.6) (width 0.2) (layer "B.Cu") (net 13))
 (segment (start 159.3977 130.4949) (end 170.2879 130.4949) (width 0.2) (layer "B.Cu") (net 13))
 (segment (start 168.8974 58.379) (end 170.5665 58.379) (width 0.2) (layer "B.Cu") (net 13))
 (segment (start 158.675 129.7722) (end 159.3977 130.4949) (width 0.2) (layer "B.Cu") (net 13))
 (segment (start 170.2879 130.4949) (end 171.7886 128.9942) (width 0.2) (layer "B.Cu") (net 13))
 (segment (start 166.5875 61.1) (end 163.2297 61.1) (width 0.2) (layer "B.Cu") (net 10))
 (segment (start 162.3942 60.2645) (end 143.2678 60.2645) (width 0.2) (layer "B.Cu") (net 10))
 (segment (start 143.2678 60.2645) (end 142.4783 59.475) (width 0.2) (layer "B.Cu") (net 10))
 (segment (start 163.2297 61.1) (end 162.3942 60.2645) (width 0.2) (layer "B.Cu") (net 10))
 (segment (start 142.4783 59.475) (end 137.1625 59.475) (width 0.2) (layer "B.Cu") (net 10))
 (segment (start 145.7678 65.6463) (end 145.7678 84.8597) (width 0.2) (layer "F.Cu") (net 4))
 (segment (start 144.33 64.2085) (end 143.495 64.2085) (width 0.2) (layer "F.Cu") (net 4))
 (segment (start 144.33 64.2085) (end 145.7678 65.6463) (width 0.2) (layer "F.Cu") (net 4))
 (via (at 145.7678 84.8597) (size 0.6) (drill 0.3) (layers "F.Cu" "B.Cu") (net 4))
 (segment (start 145.7678 84.8597) (end 147.8331 86.925) (width 0.2) (layer "B.Cu") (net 4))
 (segment (start 147.8331 86.925) (end 169.49 86.925) (width 0.2) (layer "B.Cu") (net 4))
 (segment (start 144.33 66.7485) (end 143.495 66.7485) (width 0.2) (layer "F.Cu") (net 3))
 (segment (start 161.9665 84.385) (end 169.49 84.385) (width 0.2) (layer "B.Cu") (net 3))
 (segment (start 144.33 66.7485) (end 161.9665 84.385) (width 0.2) (layer "B.Cu") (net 3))
 (segment (start 168.6755 80.6933) (end 169.49 80.6933) (width 0.2) (layer "F.Cu") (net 2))
 (segment (start 160.405 59.1285) (end 168.1002 66.8237) (width 0.2) (layer "F.Cu") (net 2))
 (segment (start 169.49 81.845) (end 169.49 80.6933) (width 0.2) (layer "F.Cu") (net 2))
 (segment (start 168.1002 66.8237) (end 168.1002 80.118) (width 0.2) (layer "F.Cu") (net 2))
 (segment (start 159.57 59.1285) (end 160.405 59.1285) (width 0.2) (layer "F.Cu") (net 2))
 (segment (start 168.1002 80.118) (end 168.6755 80.6933) (width 0.2) (layer "F.Cu") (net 2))
 (segment (start 160.405 69.2885) (end 159.57 69.2885) (width 0.2) (layer "F.Cu") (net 12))
 (segment (start 157.3326 71.5259) (end 159.57 69.2885) (width 0.2) (layer "F.Cu") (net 12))
 (segment (start 157.3326 100.5137) (end 157.3326 71.5259) (width 0.2) (layer "F.Cu") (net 12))
 (via (at 157.3326 100.5137) (size 0.6) (drill 0.3) (layers "F.Cu" "B.Cu") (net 12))
 (segment (start 138.575 102.425) (end 139.7898 101.2102) (width 0.2) (layer "B.Cu") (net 12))
 (segment (start 139.7898 101.2102) (end 144.0896 101.2102) (width 0.2) (layer "B.Cu") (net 12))
 (segment (start 144.1827 101.3033) (end 156.543 101.3033) (width 0.2) (layer "B.Cu") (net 12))
 (segment (start 156.543 101.3033) (end 157.3326 100.5137) (width 0.2) (layer "B.Cu") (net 12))
 (segment (start 144.0896 101.2102) (end 144.1827 101.3033) (width 0.2) (layer "B.Cu") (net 12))
 (segment (start 157.625 102.425) (end 156.7169 101.5169) (width 0.2) (layer "F.Cu") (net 15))
 (segment (start 156.7169 101.5169) (end 156.7169 69.6016) (width 0.2) (layer "F.Cu") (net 15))
 (segment (start 156.7169 69.6016) (end 159.57 66.7485) (width 0.2) (layer "F.Cu") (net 15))
 (segment (start 159.57 66.7485) (end 160.405 66.7485) (width 0.2) (layer "F.Cu") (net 15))
 (segment (start 159.57 64.2085) (end 160.405 64.2085) (width 0.2) (layer "F.Cu") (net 14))
 (segment (start 138.56 121.455) (end 135.8627 118.7577) (width 0.2) (layer "F.Cu") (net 14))
 (segment (start 135.8627 71.3286) (end 139.9854 67.2059) (width 0.2) (layer "F.Cu") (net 14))
 (segment (start 135.8627 118.7577) (end 135.8627 71.3286) (width 0.2) (layer "F.Cu") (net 14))
 (via (at 139.9854 67.2059) (size 0.6) (drill 0.3) (layers "F.Cu" "B.Cu") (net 14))
 (segment (start 139.9854 67.2059) (end 141.7128 65.4785) (width 0.2) (layer "B.Cu") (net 14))
 (segment (start 158.3 65.4785) (end 159.57 64.2085) (width 0.2) (layer "B.Cu") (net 14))
 (segment (start 141.7128 65.4785) (end 158.3 65.4785) (width 0.2) (layer "B.Cu") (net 14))
 (segment (start 157.625 121.425) (end 154.9308 118.7308) (width 0.2) (layer "F.Cu") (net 5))
 (segment (start 160.405 61.6685) (end 159.57 61.6685) (width 0.2) (layer "F.Cu") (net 5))
 (segment (start 154.9308 66.3077) (end 159.57 61.6685) (width 0.2) (layer "F.Cu") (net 5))
 (segment (start 154.9308 118.7308) (end 154.9308 66.3077) (width 0.2) (layer "F.Cu") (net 5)))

